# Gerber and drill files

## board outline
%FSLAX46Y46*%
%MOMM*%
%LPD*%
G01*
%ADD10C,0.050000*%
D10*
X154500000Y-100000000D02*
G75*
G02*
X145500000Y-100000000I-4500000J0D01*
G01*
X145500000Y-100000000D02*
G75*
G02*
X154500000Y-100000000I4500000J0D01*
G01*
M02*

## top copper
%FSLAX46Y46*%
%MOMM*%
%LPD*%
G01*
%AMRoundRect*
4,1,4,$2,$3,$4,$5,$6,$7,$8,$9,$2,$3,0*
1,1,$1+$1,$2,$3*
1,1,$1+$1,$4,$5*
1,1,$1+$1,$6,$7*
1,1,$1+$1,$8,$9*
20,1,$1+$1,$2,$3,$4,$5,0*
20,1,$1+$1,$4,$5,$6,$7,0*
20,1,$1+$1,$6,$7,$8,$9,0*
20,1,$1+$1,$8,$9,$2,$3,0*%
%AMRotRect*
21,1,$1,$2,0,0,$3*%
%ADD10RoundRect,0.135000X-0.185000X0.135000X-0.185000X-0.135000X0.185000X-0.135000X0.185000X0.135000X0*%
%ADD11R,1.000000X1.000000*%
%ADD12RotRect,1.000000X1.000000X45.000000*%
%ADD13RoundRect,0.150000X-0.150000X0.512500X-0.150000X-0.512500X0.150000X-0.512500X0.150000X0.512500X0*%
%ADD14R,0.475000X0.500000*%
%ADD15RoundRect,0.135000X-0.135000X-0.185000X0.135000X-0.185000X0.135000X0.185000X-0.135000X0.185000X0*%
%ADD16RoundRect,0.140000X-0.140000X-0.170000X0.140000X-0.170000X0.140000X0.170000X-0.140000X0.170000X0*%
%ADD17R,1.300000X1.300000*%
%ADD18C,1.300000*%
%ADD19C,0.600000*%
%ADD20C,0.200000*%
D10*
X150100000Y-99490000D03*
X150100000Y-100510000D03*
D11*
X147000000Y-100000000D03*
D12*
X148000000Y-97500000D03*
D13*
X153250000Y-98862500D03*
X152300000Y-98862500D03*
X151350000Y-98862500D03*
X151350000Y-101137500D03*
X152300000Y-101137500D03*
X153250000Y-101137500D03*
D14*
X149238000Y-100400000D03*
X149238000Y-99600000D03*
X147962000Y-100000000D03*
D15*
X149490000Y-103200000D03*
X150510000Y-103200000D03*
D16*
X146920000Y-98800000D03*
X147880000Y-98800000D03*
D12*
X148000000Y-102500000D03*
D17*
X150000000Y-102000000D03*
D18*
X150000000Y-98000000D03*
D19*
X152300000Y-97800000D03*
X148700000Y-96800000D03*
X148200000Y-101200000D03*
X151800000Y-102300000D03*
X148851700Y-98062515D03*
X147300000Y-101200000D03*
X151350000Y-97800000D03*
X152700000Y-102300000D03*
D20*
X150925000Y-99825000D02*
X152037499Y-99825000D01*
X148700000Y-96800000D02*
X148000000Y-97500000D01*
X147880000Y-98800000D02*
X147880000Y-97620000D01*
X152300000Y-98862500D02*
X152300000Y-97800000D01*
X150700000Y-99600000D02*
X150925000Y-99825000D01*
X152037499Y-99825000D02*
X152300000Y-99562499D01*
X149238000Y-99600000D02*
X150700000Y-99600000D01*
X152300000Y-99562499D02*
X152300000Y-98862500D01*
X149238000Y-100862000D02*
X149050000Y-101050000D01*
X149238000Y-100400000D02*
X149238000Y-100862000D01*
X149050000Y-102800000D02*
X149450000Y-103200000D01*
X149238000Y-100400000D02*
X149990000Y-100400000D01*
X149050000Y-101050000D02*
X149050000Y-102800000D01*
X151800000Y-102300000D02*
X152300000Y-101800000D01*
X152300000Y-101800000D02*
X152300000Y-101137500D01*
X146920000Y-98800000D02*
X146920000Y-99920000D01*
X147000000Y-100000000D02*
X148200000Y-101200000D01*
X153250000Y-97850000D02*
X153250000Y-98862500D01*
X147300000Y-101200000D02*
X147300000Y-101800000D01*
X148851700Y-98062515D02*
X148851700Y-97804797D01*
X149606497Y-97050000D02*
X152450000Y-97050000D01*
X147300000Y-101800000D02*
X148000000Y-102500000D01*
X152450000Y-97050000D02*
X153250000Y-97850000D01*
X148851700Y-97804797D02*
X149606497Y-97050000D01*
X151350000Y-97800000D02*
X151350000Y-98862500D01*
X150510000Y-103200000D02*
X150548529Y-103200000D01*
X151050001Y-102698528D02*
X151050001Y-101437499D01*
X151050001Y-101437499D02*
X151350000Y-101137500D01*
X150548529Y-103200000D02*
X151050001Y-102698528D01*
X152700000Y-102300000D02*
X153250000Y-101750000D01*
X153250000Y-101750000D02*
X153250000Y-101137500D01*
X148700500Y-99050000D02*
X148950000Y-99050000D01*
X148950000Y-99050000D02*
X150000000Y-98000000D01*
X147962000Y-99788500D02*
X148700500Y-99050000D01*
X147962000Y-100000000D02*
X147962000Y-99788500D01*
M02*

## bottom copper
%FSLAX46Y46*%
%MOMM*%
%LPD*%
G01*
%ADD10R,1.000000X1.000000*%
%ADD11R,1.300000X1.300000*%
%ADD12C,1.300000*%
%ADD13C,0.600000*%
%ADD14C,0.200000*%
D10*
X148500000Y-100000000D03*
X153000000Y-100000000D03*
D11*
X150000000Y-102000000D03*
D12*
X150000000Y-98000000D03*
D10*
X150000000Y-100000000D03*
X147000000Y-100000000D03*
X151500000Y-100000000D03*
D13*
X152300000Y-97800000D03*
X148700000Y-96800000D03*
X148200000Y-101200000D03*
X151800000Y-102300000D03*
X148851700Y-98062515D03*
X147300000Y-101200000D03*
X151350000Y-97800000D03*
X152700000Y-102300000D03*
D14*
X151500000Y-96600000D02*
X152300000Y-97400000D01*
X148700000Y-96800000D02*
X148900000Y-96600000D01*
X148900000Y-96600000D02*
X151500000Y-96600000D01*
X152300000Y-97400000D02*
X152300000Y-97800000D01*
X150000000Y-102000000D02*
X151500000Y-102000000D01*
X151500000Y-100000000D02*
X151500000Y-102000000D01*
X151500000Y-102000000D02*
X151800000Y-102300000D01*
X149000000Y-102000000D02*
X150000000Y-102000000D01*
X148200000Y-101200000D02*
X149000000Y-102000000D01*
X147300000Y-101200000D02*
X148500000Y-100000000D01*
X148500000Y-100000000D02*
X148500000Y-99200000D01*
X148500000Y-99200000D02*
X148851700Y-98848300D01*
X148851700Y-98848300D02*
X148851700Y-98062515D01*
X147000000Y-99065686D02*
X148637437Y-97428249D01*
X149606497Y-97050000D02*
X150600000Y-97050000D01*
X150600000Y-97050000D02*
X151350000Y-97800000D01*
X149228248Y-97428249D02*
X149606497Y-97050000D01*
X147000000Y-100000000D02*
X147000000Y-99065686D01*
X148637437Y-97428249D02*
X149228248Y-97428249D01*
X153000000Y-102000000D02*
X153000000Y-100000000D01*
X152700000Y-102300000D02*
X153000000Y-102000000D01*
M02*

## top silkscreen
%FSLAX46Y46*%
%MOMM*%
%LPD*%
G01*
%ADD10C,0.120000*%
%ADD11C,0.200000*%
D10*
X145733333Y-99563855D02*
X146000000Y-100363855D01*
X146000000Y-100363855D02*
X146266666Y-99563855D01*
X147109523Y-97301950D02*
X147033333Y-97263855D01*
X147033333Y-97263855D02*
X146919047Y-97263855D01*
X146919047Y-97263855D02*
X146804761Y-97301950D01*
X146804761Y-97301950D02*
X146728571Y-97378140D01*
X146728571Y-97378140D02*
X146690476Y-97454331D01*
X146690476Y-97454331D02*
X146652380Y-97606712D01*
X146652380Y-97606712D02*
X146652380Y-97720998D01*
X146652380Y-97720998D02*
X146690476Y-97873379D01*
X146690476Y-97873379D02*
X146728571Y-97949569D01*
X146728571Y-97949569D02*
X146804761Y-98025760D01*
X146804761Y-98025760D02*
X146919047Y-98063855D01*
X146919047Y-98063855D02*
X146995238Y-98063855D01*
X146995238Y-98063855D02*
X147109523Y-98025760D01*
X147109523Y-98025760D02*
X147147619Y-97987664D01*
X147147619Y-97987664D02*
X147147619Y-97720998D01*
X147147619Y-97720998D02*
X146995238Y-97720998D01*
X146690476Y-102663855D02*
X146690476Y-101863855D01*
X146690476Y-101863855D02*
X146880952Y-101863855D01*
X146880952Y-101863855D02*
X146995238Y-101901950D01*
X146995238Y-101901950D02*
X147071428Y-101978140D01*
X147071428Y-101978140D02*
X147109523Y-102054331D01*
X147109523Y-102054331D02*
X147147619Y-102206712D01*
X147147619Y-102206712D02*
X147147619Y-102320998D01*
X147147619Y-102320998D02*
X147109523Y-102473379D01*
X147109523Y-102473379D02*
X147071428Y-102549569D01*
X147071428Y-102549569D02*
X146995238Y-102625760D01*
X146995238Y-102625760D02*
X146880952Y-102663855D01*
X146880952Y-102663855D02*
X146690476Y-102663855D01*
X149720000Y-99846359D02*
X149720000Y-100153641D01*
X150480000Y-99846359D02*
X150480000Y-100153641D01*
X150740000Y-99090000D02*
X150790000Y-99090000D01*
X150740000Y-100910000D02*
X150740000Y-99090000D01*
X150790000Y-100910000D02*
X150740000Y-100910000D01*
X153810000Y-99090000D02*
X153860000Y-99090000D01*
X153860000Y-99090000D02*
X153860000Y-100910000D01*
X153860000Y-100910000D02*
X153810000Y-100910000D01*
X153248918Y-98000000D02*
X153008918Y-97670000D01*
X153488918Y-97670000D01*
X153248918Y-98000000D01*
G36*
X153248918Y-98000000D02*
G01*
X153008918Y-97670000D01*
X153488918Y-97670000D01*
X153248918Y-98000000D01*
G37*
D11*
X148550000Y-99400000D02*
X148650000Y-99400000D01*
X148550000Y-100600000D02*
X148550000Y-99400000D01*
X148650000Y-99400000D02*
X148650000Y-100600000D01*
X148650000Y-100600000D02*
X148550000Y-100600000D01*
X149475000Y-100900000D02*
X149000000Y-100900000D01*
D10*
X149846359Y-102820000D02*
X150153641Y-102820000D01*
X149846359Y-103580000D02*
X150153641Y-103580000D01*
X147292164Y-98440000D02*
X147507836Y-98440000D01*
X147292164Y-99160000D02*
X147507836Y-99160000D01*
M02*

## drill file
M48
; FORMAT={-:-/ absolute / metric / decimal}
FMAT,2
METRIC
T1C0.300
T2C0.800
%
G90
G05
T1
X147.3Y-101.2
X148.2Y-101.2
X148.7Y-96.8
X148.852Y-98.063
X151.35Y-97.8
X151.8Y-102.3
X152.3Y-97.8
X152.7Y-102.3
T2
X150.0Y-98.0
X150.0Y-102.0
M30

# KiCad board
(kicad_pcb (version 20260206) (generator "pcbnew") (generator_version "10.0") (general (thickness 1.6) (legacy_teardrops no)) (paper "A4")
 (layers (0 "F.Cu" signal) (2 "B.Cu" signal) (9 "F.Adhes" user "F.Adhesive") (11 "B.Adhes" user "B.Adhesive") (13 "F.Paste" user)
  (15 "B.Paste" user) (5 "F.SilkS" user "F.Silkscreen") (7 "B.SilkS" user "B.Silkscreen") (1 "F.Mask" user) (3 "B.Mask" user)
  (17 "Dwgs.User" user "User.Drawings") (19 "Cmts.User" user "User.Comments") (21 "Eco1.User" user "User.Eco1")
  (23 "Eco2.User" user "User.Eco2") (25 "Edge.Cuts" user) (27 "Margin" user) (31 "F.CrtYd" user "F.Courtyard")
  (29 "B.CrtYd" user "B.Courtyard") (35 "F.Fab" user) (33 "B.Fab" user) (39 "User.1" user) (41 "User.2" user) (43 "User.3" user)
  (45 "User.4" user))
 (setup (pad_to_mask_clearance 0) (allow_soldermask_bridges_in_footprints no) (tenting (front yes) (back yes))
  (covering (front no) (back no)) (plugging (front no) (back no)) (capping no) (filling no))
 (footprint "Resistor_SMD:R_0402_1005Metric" (layer "F.Cu") (at 150.1 100 -90)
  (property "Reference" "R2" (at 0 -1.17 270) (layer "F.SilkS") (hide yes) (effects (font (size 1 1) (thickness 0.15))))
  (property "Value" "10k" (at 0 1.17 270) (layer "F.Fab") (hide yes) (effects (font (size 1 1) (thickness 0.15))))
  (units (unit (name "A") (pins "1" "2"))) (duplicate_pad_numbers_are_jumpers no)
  (fp_line (start -0.153641 0.38) (end 0.153641 0.38) (stroke (width 0.12) (type solid)) (layer "F.SilkS"))
  (fp_line (start -0.153641 -0.38) (end 0.153641 -0.38) (stroke (width 0.12) (type solid)) (layer "F.SilkS"))
  (pad "1" smd roundrect (at -0.51 0 270) (size 0.54 0.64) (layers "F.Cu" "F.Mask" "F.Paste") (roundrect_rratio 0.25) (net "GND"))
  (pad "2" smd roundrect (at 0.51 0 270) (size 0.54 0.64) (layers "F.Cu" "F.Mask" "F.Paste") (roundrect_rratio 0.25) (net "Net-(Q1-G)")))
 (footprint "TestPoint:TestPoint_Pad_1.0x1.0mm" (layer "F.Cu") (at 147 100)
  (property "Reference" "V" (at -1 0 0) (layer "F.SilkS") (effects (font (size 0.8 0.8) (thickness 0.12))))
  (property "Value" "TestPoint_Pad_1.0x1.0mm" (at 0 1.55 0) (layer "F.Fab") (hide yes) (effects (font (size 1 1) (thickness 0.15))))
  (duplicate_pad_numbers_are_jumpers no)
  (pad "1" smd rect (at 0 0) (size 1 1) (layers "F.Cu" "F.Mask") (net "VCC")))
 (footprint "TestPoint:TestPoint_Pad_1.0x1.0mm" (layer "F.Cu") (at 148 97.5 45)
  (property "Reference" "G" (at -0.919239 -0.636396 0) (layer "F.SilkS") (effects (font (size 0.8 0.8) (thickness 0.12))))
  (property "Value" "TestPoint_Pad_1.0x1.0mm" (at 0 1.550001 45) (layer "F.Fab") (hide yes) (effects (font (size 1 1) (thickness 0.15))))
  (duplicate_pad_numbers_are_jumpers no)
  (pad "1" smd rect (at 0 0 45) (size 1 1) (layers "F.Cu" "F.Mask") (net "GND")))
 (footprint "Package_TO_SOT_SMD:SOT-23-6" (layer "F.Cu") (at 152.3 100 -90)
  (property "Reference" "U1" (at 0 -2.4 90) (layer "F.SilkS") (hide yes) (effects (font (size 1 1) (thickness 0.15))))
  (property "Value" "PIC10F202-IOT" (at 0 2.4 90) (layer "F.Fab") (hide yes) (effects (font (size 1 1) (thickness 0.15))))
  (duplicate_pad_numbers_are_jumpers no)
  (fp_line (start -0.91 1.56) (end -0.91 1.51) (stroke (width 0.12) (type solid)) (layer "F.SilkS"))
  (fp_line (start 0.91 1.56) (end -0.91 1.56) (stroke (width 0.12) (type solid)) (layer "F.SilkS"))
  (fp_line (start 0.91 1.51) (end 0.91 1.56) (stroke (width 0.12) (type solid)) (layer "F.SilkS"))
  (fp_line (start -0.91 -1.51) (end -0.91 -1.56) (stroke (width 0.12) (type solid)) (layer "F.SilkS"))
  (fp_line (start -0.91 -1.56) (end 0.91 -1.56) (stroke (width 0.12) (type solid)) (layer "F.SilkS"))
  (fp_line (start 0.91 -1.56) (end 0.91 -1.51) (stroke (width 0.12) (type solid)) (layer "F.SilkS"))
  (fp_poly
   (pts (xy -2 -0.948918) (xy -2.33 -0.708918) (xy -2.33 -1.188918)) (stroke (width 0.12) (type solid)) (fill yes) (layer "F.SilkS"))
  (pad "1" smd roundrect (at -1.1375 -0.95 270) (size 1.325 0.6) (layers "F.Cu" "F.Mask" "F.Paste") (roundrect_rratio 0.25) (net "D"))
  (pad "2" smd roundrect (at -1.1375 0 270) (size 1.325 0.6) (layers "F.Cu" "F.Mask" "F.Paste") (roundrect_rratio 0.25) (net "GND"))
  (pad "3" smd roundrect (at -1.1375 0.95 270) (size 1.325 0.6) (layers "F.Cu" "F.Mask" "F.Paste") (roundrect_rratio 0.25) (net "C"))
  (pad "4" smd roundrect (at 1.1375 0.95 270) (size 1.325 0.6) (layers "F.Cu" "F.Mask" "F.Paste") (roundrect_rratio 0.25)
   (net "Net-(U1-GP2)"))
  (pad "5" smd roundrect (at 1.1375 0 270) (size 1.325 0.6) (layers "F.Cu" "F.Mask" "F.Paste") (roundrect_rratio 0.25) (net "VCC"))
  (pad "6" smd roundrect (at 1.1375 -0.95 270) (size 1.325 0.6) (layers "F.Cu" "F.Mask" "F.Paste") (roundrect_rratio 0.25) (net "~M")))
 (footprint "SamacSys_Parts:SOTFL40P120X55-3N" (layer "F.Cu") (at 148.6 100 180)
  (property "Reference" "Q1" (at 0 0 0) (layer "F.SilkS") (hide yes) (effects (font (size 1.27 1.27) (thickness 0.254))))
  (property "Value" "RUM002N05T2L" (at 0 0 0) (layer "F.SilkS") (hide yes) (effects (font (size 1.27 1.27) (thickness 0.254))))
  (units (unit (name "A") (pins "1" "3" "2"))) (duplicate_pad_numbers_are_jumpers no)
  (fp_line (start 0.05 0.6) (end -0.05 0.6) (stroke (width 0.2) (type solid)) (layer "F.SilkS"))
  (fp_line (start 0.05 -0.6) (end 0.05 0.6) (stroke (width 0.2) (type solid)) (layer "F.SilkS"))
  (fp_line (start -0.05 0.6) (end -0.05 -0.6) (stroke (width 0.2) (type solid)) (layer "F.SilkS"))
  (fp_line (start -0.05 -0.6) (end 0.05 -0.6) (stroke (width 0.2) (type solid)) (layer "F.SilkS"))
  (fp_line (start -0.875 -0.9) (end -0.4 -0.9) (stroke (width 0.2) (type solid)) (layer "F.SilkS"))
  (pad "1" smd rect (at -0.638 -0.4 180) (size 0.475 0.5) (layers "F.Cu" "F.Mask" "F.Paste") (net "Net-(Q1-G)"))
  (pad "2" smd rect (at -0.638 0.4 180) (size 0.475 0.5) (layers "F.Cu" "F.Mask" "F.Paste") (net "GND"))
  (pad "3" smd rect (at 0.638 0 180) (size 0.475 0.5) (layers "F.Cu" "F.Mask" "F.Paste") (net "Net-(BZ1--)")))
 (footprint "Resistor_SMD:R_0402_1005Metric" (layer "F.Cu") (at 150 103.2)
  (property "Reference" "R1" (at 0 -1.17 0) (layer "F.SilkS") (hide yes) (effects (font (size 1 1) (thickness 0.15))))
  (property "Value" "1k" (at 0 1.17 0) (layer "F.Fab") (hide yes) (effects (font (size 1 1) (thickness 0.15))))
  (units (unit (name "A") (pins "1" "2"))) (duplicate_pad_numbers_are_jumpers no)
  (fp_line (start -0.153641 -0.38) (end 0.153641 -0.38) (stroke (width 0.12) (type solid)) (layer "F.SilkS"))
  (fp_line (start -0.153641 0.38) (end 0.153641 0.38) (stroke (width 0.12) (type solid)) (layer "F.SilkS"))
  (pad "1" smd roundrect (at -0.51 0) (size 0.54 0.64) (layers "F.Cu" "F.Mask" "F.Paste") (roundrect_rratio 0.25) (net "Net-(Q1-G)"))
  (pad "2" smd roundrect (at 0.51 0) (size 0.54 0.64) (layers "F.Cu" "F.Mask" "F.Paste") (roundrect_rratio 0.25) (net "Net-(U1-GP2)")))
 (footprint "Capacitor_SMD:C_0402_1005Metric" (layer "F.Cu") (at 147.4 98.8)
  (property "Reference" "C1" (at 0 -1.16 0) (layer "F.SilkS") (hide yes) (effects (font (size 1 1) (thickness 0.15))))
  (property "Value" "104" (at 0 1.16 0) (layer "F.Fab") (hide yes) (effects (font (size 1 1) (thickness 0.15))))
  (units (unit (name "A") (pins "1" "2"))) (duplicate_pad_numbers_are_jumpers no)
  (fp_line (start -0.107836 -0.36) (end 0.107836 -0.36) (stroke (width 0.12) (type solid)) (layer "F.SilkS"))
  (fp_line (start -0.107836 0.36) (end 0.107836 0.36) (stroke (width 0.12) (type solid)) (layer "F.SilkS"))
  (pad "1" smd roundrect (at -0.48 0) (size 0.56 0.62) (layers "F.Cu" "F.Mask" "F.Paste") (roundrect_rratio 0.25) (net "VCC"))
  (pad "2" smd roundrect (at 0.48 0) (size 0.56 0.62) (layers "F.Cu" "F.Mask" "F.Paste") (roundrect_rratio 0.25) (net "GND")))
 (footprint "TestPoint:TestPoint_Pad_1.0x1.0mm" (layer "F.Cu") (at 148 102.5 45)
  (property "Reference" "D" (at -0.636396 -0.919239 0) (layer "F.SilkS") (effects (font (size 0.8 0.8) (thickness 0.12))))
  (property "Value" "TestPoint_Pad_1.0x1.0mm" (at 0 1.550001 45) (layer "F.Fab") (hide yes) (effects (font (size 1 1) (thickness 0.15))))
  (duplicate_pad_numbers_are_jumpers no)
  (pad "1" smd rect (at 0 0 45) (size 1 1) (layers "F.Cu" "F.Mask") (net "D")))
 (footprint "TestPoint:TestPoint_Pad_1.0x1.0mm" (layer "B.Cu") (at 148.5 100)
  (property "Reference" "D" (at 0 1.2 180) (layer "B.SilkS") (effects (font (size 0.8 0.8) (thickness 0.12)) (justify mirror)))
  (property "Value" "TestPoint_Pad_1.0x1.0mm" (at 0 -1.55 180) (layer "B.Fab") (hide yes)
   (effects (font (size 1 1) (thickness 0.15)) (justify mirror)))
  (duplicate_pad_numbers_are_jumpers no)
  (pad "1" smd rect (at 0 0) (size 1 1) (layers "B.Cu" "B.Mask") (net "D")))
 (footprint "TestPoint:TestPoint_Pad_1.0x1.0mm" (layer "B.Cu") (at 153 100)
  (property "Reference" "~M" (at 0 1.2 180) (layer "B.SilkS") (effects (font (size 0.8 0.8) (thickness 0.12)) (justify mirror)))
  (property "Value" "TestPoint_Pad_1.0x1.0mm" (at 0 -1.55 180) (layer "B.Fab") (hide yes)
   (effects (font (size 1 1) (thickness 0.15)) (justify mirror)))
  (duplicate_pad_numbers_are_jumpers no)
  (pad "1" smd rect (at 0 0) (size 1 1) (layers "B.Cu" "B.Mask") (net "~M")))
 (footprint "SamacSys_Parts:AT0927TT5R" (layer "B.Cu") (at 150 102 180)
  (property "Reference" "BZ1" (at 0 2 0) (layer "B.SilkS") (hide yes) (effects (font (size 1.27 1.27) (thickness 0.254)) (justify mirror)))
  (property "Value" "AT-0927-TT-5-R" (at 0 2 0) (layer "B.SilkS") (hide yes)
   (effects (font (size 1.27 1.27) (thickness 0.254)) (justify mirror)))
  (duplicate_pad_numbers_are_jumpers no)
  (pad "1" thru_hole rect (at 0 0 180) (size 1.3 1.3) (drill 0.8) (layers "*.Cu" "*.Mask") (remove_unused_layers no) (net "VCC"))
  (pad "2" thru_hole circle (at 0 4 180) (size 1.3 1.3) (drill 0.8) (layers "*.Cu" "*.Mask") (remove_unused_layers no) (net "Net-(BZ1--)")))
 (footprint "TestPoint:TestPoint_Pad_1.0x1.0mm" (layer "B.Cu") (at 150 100)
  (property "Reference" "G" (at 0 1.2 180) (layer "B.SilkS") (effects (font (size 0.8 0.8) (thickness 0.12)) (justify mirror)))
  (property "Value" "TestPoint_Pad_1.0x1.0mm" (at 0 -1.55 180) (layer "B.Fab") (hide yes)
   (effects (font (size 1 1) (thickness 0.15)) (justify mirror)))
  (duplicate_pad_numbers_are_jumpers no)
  (pad "1" smd rect (at 0 0) (size 1 1) (layers "B.Cu" "B.Mask")))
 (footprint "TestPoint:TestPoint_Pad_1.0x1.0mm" (layer "B.Cu") (at 147 100)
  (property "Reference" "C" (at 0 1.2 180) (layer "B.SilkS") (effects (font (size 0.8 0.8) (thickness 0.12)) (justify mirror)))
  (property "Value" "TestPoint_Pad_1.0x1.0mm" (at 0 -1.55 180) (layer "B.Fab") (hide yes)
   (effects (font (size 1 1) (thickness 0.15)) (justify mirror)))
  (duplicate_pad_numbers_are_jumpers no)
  (pad "1" smd rect (at 0 0) (size 1 1) (layers "B.Cu" "B.Mask") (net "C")))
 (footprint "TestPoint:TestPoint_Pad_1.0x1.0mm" (layer "B.Cu") (at 151.5 100)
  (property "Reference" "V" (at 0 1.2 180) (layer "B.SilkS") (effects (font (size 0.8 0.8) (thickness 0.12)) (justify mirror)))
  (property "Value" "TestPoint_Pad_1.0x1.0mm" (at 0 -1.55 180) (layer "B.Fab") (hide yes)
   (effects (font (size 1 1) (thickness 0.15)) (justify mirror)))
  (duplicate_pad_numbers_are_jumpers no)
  (pad "1" smd rect (at 0 0) (size 1 1) (layers "B.Cu" "B.Mask") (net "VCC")))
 (gr_circle (center 150 100) (end 154.5 100) (stroke (width 0.05) (type default)) (fill no) (layer "Edge.Cuts"))
 (segment (start 150.925 99.825) (end 152.037499 99.825) (width 0.2) (layer "F.Cu") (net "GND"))
 (segment (start 148.7 96.8) (end 148 97.5) (width 0.2) (layer "F.Cu") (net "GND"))
 (segment (start 147.88 98.8) (end 147.88 97.62) (width 0.2) (layer "F.Cu") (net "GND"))
 (segment (start 152.3 98.8625) (end 152.3 97.8) (width 0.2) (layer "F.Cu") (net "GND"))
 (segment (start 150.7 99.6) (end 150.925 99.825) (width 0.2) (layer "F.Cu") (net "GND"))
 (segment (start 152.037499 99.825) (end 152.3 99.562499) (width 0.2) (layer "F.Cu") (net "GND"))
 (segment (start 149.238 99.6) (end 150.7 99.6) (width 0.2) (layer "F.Cu") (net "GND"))
 (segment (start 152.3 99.562499) (end 152.3 98.8625) (width 0.2) (layer "F.Cu") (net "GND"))
 (via (at 152.3 97.8) (size 0.6) (drill 0.3) (layers "F.Cu" "B.Cu") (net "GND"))
 (via (at 148.7 96.8) (size 0.6) (drill 0.3) (layers "F.Cu" "B.Cu") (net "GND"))
 (segment (start 151.5 96.6) (end 152.3 97.4) (width 0.2) (layer "B.Cu") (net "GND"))
 (segment (start 148.7 96.8) (end 148.9 96.6) (width 0.2) (layer "B.Cu") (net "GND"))
 (segment (start 148.9 96.6) (end 151.5 96.6) (width 0.2) (layer "B.Cu") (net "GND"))
 (segment (start 152.3 97.4) (end 152.3 97.8) (width 0.2) (layer "B.Cu") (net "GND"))
 (segment (start 149.238 100.862) (end 149.05 101.05) (width 0.2) (layer "F.Cu") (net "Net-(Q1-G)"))
 (segment (start 149.238 100.4) (end 149.238 100.862) (width 0.2) (layer "F.Cu") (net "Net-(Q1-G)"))
 (segment (start 149.05 102.8) (end 149.45 103.2) (width 0.2) (layer "F.Cu") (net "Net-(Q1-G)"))
 (segment (start 149.238 100.4) (end 149.99 100.4) (width 0.2) (layer "F.Cu") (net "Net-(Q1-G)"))
 (segment (start 149.05 101.05) (end 149.05 102.8) (width 0.2) (layer "F.Cu") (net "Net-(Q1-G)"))
 (segment (start 151.8 102.3) (end 152.3 101.8) (width 0.2) (layer "F.Cu") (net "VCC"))
 (segment (start 152.3 101.8) (end 152.3 101.1375) (width 0.2) (layer "F.Cu") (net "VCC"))
 (segment (start 146.92 98.8) (end 146.92 99.92) (width 0.2) (layer "F.Cu") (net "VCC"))
 (segment (start 147 100) (end 148.2 101.2) (width 0.2) (layer "F.Cu") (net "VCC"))
 (via (at 148.2 101.2) (size 0.6) (drill 0.3) (layers "F.Cu" "B.Cu") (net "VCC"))
 (via (at 151.8 102.3) (size 0.6) (drill 0.3) (layers "F.Cu" "B.Cu") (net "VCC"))
 (segment (start 150 102) (end 151.5 102) (width 0.2) (layer "B.Cu") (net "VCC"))
 (segment (start 151.5 100) (end 151.5 102) (width 0.2) (layer "B.Cu") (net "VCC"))
 (segment (start 151.5 102) (end 151.8 102.3) (width 0.2) (layer "B.Cu") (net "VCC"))
 (segment (start 149 102) (end 150 102) (width 0.2) (layer "B.Cu") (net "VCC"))
 (segment (start 148.2 101.2) (end 149 102) (width 0.2) (layer "B.Cu") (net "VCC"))
 (segment (start 153.25 97.85) (end 153.25 98.8625) (width 0.2) (layer "F.Cu") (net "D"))
 (segment (start 147.3 101.2) (end 147.3 101.8) (width 0.2) (layer "F.Cu") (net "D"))
 (segment (start 148.8517 98.062515) (end 148.8517 97.804797) (width 0.2) (layer "F.Cu") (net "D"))
 (segment (start 149.606497 97.05) (end 152.45 97.05) (width 0.2) (layer "F.Cu") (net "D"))
 (segment (start 147.3 101.8) (end 148 102.5) (width 0.2) (layer "F.Cu") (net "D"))
 (segment (start 152.45 97.05) (end 153.25 97.85) (width 0.2) (layer "F.Cu") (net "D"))
 (segment (start 148.8517 97.804797) (end 149.606497 97.05) (width 0.2) (layer "F.Cu") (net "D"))
 (via (at 148.8517 98.062515) (size 0.6) (drill 0.3) (layers "F.Cu" "B.Cu") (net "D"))
 (via (at 147.3 101.2) (size 0.6) (drill 0.3) (layers "F.Cu" "B.Cu") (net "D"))
 (segment (start 147.3 101.2) (end 148.5 100) (width 0.2) (layer "B.Cu") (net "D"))
 (segment (start 148.5 100) (end 148.5 99.2) (width 0.2) (layer "B.Cu") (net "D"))
 (segment (start 148.5 99.2) (end 148.8517 98.8483) (width 0.2) (layer "B.Cu") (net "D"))
 (segment (start 148.8517 98.8483) (end 148.8517 98.062515) (width 0.2) (layer "B.Cu") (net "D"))
 (segment (start 151.35 97.8) (end 151.35 98.8625) (width 0.2) (layer "F.Cu") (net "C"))
 (via (at 151.35 97.8) (size 0.6) (drill 0.3) (layers "F.Cu" "B.Cu") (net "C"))
 (segment (start 147 99.065686) (end 148.637437 97.428249) (width 0.2) (layer "B.Cu") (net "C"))
 (segment (start 149.606497 97.05) (end 150.6 97.05) (width 0.2) (layer "B.Cu") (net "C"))
 (segment (start 150.6 97.05) (end 151.35 97.8) (width 0.2) (layer "B.Cu") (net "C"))
 (segment (start 149.228248 97.428249) (end 149.606497 97.05) (width 0.2) (layer "B.Cu") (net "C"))
 (segment (start 147 100) (end 147 99.065686) (width 0.2) (layer "B.Cu") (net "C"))
 (segment (start 148.637437 97.428249) (end 149.228248 97.428249) (width 0.2) (layer "B.Cu") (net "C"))
 (segment (start 150.51 103.2) (end 150.548529 103.2) (width 0.2) (layer "F.Cu") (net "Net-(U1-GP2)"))
 (segment (start 151.050001 102.698528) (end 151.050001 101.437499) (width 0.2) (layer "F.Cu") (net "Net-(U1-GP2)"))
 (segment (start 151.050001 101.437499) (end 151.35 101.1375) (width 0.2) (layer "F.Cu") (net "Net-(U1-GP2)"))
 (segment (start 150.548529 103.2) (end 151.050001 102.698528) (width 0.2) (layer "F.Cu") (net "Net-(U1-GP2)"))
 (segment (start 152.7 102.3) (end 153.25 101.75) (width 0.2) (layer "F.Cu") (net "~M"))
 (segment (start 153.25 101.75) (end 153.25 101.1375) (width 0.2) (layer "F.Cu") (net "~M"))
 (via (at 152.7 102.3) (size 0.6) (drill 0.3) (layers "F.Cu" "B.Cu") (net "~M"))
 (segment (start 153 102) (end 153 100) (width 0.2) (layer "B.Cu") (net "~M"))
 (segment (start 152.7 102.3) (end 153 102) (width 0.2) (layer "B.Cu") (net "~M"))
 (segment (start 148.7005 99.05) (end 148.95 99.05) (width 0.2) (layer "F.Cu") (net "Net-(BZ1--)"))
 (segment (start 148.95 99.05) (end 150 98) (width 0.2) (layer "F.Cu") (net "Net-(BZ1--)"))
 (segment (start 147.962 99.7885) (end 148.7005 99.05) (width 0.2) (layer "F.Cu") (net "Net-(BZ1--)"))
 (segment (start 147.962 100) (end 147.962 99.7885) (width 0.2) (layer "F.Cu") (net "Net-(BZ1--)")))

